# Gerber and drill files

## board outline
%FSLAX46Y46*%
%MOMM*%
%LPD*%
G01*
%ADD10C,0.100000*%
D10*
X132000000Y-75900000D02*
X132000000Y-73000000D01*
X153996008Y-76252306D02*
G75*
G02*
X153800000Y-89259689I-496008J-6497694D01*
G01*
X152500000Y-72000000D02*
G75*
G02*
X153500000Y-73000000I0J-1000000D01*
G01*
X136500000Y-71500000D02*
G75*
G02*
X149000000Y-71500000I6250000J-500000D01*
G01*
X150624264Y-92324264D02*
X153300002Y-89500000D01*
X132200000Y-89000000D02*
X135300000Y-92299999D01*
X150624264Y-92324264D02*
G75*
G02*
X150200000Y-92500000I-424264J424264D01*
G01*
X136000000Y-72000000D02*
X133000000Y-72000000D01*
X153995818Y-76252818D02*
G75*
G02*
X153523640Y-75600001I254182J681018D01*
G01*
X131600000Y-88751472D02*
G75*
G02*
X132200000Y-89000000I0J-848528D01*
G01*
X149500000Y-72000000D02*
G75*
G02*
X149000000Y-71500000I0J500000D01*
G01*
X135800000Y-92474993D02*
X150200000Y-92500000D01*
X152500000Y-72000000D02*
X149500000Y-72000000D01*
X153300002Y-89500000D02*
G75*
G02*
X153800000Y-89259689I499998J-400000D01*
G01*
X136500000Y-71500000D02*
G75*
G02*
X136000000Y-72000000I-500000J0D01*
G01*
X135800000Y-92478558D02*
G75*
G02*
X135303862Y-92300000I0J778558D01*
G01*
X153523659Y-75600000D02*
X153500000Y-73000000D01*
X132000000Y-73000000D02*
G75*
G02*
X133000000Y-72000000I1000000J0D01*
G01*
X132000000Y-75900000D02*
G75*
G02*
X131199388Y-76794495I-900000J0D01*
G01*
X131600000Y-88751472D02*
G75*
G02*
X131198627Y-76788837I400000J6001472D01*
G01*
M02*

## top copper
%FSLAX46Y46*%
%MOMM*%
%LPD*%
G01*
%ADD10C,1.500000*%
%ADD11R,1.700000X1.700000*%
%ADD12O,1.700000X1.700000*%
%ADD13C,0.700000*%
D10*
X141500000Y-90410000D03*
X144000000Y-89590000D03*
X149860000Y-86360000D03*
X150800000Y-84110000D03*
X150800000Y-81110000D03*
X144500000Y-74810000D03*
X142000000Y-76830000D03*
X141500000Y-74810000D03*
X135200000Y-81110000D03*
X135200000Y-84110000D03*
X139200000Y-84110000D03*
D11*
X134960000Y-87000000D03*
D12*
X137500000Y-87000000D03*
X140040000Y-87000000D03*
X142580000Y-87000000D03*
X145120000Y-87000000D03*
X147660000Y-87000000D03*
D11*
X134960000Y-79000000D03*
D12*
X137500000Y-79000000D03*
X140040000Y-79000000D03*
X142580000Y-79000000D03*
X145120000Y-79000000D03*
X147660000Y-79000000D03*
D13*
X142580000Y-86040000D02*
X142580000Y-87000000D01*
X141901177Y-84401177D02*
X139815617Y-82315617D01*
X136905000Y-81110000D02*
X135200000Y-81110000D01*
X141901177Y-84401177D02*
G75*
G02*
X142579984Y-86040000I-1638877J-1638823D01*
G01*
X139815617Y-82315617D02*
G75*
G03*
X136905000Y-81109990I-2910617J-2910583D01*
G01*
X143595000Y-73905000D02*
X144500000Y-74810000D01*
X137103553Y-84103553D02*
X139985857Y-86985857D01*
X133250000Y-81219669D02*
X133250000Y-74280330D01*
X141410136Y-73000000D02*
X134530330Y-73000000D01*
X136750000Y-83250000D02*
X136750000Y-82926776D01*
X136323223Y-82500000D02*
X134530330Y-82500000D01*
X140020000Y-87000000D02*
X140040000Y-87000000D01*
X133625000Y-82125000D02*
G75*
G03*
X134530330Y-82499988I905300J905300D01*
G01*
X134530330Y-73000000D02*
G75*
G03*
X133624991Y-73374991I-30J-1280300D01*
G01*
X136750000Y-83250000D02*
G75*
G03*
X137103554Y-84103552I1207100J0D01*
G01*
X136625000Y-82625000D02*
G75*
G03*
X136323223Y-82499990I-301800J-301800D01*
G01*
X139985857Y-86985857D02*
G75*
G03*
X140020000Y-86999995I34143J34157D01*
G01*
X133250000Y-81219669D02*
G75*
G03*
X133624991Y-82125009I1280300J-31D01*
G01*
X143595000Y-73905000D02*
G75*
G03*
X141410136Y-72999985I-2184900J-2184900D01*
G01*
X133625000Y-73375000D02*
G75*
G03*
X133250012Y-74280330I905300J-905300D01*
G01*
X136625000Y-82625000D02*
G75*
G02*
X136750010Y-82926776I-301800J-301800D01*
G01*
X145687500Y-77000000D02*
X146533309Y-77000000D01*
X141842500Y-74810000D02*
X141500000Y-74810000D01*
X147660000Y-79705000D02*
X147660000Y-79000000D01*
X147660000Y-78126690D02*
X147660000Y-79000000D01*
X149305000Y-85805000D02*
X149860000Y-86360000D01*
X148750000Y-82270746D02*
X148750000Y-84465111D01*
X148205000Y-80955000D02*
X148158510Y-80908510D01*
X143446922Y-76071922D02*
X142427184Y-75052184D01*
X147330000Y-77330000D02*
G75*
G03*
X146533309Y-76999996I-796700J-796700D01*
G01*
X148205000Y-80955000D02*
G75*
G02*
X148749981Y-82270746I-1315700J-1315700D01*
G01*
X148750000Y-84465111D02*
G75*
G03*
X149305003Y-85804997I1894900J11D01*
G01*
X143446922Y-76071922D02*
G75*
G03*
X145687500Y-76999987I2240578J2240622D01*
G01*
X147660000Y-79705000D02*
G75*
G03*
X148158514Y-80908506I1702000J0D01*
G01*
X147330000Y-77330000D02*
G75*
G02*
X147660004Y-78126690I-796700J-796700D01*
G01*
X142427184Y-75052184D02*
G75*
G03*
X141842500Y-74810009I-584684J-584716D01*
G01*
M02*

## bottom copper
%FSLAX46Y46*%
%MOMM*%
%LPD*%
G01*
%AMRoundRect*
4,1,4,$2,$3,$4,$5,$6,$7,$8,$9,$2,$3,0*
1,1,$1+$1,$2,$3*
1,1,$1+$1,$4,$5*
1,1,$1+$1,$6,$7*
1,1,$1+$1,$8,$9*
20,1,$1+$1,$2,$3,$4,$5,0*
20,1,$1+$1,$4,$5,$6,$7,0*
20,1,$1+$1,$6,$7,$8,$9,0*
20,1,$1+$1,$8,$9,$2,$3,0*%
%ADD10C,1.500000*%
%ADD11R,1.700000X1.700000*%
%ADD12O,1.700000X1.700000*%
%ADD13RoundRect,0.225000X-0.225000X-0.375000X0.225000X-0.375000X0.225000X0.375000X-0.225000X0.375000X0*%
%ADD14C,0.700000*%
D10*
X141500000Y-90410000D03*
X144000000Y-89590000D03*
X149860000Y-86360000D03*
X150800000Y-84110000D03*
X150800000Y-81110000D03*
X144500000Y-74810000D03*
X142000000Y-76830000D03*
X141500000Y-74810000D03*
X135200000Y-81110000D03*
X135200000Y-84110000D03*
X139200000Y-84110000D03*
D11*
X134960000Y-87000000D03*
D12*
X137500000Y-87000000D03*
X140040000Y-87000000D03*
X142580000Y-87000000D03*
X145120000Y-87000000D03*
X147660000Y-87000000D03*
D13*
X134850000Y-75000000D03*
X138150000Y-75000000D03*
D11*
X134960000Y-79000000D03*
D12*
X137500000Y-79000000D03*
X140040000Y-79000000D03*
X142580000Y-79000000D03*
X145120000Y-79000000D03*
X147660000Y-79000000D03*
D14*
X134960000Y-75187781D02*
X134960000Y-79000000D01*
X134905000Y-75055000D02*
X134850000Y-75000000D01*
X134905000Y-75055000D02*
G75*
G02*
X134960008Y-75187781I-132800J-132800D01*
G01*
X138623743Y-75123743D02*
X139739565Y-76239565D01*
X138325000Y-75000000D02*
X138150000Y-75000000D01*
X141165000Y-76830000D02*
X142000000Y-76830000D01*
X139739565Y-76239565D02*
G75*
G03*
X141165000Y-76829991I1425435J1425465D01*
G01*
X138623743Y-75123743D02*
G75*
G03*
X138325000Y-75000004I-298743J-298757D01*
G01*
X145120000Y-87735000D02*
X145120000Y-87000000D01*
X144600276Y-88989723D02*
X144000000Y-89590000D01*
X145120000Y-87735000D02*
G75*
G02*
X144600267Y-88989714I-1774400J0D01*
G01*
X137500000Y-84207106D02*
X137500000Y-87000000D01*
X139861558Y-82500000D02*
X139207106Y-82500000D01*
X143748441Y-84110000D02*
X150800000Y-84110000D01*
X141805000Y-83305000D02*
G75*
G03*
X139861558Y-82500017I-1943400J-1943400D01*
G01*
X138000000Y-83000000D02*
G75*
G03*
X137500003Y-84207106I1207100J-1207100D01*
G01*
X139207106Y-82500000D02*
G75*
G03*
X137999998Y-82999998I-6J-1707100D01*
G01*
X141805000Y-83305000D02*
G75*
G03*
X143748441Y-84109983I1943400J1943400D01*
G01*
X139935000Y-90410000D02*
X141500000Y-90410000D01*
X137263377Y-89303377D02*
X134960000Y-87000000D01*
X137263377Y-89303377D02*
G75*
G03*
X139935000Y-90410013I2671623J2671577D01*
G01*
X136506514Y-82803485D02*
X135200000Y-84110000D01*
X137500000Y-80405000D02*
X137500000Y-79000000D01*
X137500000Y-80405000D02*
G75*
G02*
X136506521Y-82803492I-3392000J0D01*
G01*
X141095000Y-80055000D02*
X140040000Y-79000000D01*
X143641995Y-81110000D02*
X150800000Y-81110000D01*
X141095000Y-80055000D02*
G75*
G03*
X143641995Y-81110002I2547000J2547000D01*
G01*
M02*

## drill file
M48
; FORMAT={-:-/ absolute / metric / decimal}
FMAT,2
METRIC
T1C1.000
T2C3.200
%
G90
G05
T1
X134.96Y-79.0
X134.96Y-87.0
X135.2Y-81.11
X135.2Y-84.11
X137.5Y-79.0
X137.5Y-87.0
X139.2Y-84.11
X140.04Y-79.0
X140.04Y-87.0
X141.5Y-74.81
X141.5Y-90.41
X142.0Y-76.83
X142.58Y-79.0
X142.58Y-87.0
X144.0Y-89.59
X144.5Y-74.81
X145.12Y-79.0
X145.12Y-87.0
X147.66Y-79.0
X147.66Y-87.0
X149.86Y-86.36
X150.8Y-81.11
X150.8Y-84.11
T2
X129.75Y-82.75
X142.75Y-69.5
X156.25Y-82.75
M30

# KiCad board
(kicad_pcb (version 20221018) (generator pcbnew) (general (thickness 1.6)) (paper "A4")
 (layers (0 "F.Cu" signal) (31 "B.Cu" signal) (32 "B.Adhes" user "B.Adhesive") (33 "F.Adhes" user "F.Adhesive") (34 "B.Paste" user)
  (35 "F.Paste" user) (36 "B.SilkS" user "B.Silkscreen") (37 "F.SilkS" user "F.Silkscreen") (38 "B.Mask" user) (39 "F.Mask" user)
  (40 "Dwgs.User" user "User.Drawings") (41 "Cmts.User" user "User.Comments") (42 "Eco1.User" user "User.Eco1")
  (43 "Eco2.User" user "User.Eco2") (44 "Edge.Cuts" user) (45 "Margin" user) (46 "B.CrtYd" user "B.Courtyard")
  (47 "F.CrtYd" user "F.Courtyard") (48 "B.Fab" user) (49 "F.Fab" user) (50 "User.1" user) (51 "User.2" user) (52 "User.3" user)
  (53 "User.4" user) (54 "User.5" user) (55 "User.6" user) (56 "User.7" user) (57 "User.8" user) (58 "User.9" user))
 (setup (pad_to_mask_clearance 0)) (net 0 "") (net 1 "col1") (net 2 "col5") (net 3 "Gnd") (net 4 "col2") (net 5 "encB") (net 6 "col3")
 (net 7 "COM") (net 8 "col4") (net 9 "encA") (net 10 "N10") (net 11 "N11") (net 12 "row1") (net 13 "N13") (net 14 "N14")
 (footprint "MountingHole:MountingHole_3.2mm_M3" (layer "F.Cu") (at 129.75 82.75)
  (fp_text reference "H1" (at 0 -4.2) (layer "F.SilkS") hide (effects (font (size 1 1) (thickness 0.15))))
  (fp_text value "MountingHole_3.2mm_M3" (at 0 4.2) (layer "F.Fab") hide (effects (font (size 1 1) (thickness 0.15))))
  (pad "" np_thru_hole circle (at 0 0) (size 3.2 3.2) (drill 3.2) (layers "*.Cu" "*.Mask")))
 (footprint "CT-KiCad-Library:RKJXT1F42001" (layer "F.Cu") (at 143 82.61)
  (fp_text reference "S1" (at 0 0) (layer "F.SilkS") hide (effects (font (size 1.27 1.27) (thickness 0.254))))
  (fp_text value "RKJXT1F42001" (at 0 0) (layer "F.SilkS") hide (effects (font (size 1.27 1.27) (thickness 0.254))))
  (pad "1" thru_hole circle (at -1.5 7.8) (size 1.5 1.5) (drill 1) (layers "*.Cu" "*.Mask") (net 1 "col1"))
  (pad "2" thru_hole circle (at 1 6.98) (size 1.5 1.5) (drill 1) (layers "*.Cu" "*.Mask") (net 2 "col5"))
  (pad "3" thru_hole circle (at 6.86 3.75) (size 1.5 1.5) (drill 1) (layers "*.Cu" "*.Mask") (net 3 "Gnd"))
  (pad "4" thru_hole circle (at 7.8 1.5) (size 1.5 1.5) (drill 1) (layers "*.Cu" "*.Mask") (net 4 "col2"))
  (pad "5" thru_hole circle (at 7.8 -1.5) (size 1.5 1.5) (drill 1) (layers "*.Cu" "*.Mask") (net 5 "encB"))
  (pad "6" thru_hole circle (at 1.5 -7.8) (size 1.5 1.5) (drill 1) (layers "*.Cu" "*.Mask") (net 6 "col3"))
  (pad "7" thru_hole circle (at -1 -5.78) (size 1.5 1.5) (drill 1) (layers "*.Cu" "*.Mask") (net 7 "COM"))
  (pad "8" thru_hole circle (at -1.5 -7.8) (size 1.5 1.5) (drill 1) (layers "*.Cu" "*.Mask") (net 3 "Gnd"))
  (pad "9" thru_hole circle (at -7.8 -1.5) (size 1.5 1.5) (drill 1) (layers "*.Cu" "*.Mask") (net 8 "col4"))
  (pad "10" thru_hole circle (at -7.8 1.5) (size 1.5 1.5) (drill 1) (layers "*.Cu" "*.Mask") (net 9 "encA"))
  (pad "11" thru_hole circle (at -3.8 1.5) (size 1.5 1.5) (drill 1) (layers "*.Cu" "*.Mask") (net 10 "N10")))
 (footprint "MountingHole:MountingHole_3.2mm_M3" (layer "F.Cu") (at 142.75 69.5)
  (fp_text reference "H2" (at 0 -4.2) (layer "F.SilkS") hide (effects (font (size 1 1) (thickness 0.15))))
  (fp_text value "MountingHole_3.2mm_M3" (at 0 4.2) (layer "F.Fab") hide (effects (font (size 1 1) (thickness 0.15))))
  (pad "" np_thru_hole circle (at 0 0) (size 3.2 3.2) (drill 3.2) (layers "*.Cu" "*.Mask")))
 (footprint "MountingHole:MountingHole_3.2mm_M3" (layer "F.Cu") (at 156.25 82.75)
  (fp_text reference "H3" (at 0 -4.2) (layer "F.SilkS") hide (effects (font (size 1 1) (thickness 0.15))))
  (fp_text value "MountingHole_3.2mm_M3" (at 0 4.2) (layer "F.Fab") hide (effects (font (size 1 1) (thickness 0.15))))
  (pad "" np_thru_hole circle (at 0 0) (size 3.2 3.2) (drill 3.2) (layers "*.Cu" "*.Mask")))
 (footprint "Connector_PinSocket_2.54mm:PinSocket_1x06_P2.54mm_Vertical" (layer "B.Cu") (at 134.96 87 -90)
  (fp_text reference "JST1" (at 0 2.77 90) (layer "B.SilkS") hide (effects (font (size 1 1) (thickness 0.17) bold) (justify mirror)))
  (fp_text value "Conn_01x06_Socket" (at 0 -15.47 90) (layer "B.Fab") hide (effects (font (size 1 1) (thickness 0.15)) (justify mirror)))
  (pad "1" thru_hole rect (at 0 0 270) (size 1.7 1.7) (drill 1) (layers "*.Cu" "*.Mask") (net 1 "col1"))
  (pad "2" thru_hole oval (at 0 -2.54 270) (size 1.7 1.7) (drill 1) (layers "*.Cu" "*.Mask") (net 4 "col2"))
  (pad "3" thru_hole oval (at 0 -5.08 270) (size 1.7 1.7) (drill 1) (layers "*.Cu" "*.Mask") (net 6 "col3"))
  (pad "4" thru_hole oval (at 0 -7.62 270) (size 1.7 1.7) (drill 1) (layers "*.Cu" "*.Mask") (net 8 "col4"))
  (pad "5" thru_hole oval (at 0 -10.16 270) (size 1.7 1.7) (drill 1) (layers "*.Cu" "*.Mask") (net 2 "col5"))
  (pad "6" thru_hole oval (at 0 -12.7 270) (size 1.7 1.7) (drill 1) (layers "*.Cu" "*.Mask") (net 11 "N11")))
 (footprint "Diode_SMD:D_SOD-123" (layer "B.Cu") (at 136.5 75)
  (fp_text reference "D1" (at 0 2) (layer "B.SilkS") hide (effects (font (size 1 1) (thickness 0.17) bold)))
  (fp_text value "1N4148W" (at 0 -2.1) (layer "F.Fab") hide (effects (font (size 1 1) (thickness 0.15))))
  (pad "1" smd roundrect (at -1.65 0) (size 0.9 1.2) (layers "B.Cu" "B.Paste" "B.Mask") (roundrect_rratio 0.25) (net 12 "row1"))
  (pad "2" smd roundrect (at 1.65 0) (size 0.9 1.2) (layers "B.Cu" "B.Paste" "B.Mask") (roundrect_rratio 0.25) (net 7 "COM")))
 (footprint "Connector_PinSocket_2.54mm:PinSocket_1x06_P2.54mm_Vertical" (layer "B.Cu") (at 134.96 79 -90)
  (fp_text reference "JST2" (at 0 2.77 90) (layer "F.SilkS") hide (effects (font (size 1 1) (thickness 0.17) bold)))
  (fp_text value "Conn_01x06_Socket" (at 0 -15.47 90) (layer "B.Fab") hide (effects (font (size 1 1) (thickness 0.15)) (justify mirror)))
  (pad "1" thru_hole rect (at 0 0 270) (size 1.7 1.7) (drill 1) (layers "*.Cu" "*.Mask") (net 12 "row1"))
  (pad "2" thru_hole oval (at 0 -2.54 270) (size 1.7 1.7) (drill 1) (layers "*.Cu" "*.Mask") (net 9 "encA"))
  (pad "3" thru_hole oval (at 0 -5.08 270) (size 1.7 1.7) (drill 1) (layers "*.Cu" "*.Mask") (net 5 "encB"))
  (pad "4" thru_hole oval (at 0 -7.62 270) (size 1.7 1.7) (drill 1) (layers "*.Cu" "*.Mask") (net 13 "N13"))
  (pad "5" thru_hole oval (at 0 -10.16 270) (size 1.7 1.7) (drill 1) (layers "*.Cu" "*.Mask") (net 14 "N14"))
  (pad "6" thru_hole oval (at 0 -12.7 270) (size 1.7 1.7) (drill 1) (layers "*.Cu" "*.Mask") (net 3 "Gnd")))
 (gr_line (start 132 75.9) (end 132 73) (stroke (width 0.1) (type default)) (layer "Edge.Cuts"))
 (gr_arc (start 153.996008 76.252306) (mid 160.015858 82.848187) (end 153.8 89.259689) (stroke (width 0.1) (type default))
  (layer "Edge.Cuts"))
 (gr_arc (start 152.5 72) (mid 153.207107 72.292893) (end 153.5 73) (stroke (width 0.1) (type default)) (layer "Edge.Cuts"))
 (gr_arc (start 136.5 71.5) (mid 142.75 65.730032) (end 149 71.5) (stroke (width 0.1) (type default)) (layer "Edge.Cuts"))
 (gr_line (start 150.624264 92.324264) (end 153.300002 89.5) (stroke (width 0.1) (type default)) (layer "Edge.Cuts"))
 (gr_line (start 132.2 89) (end 135.3 92.299999) (stroke (width 0.1) (type default)) (layer "Edge.Cuts"))
 (gr_arc (start 150.624264 92.324264) (mid 150.42961 92.454328) (end 150.2 92.5) (stroke (width 0.1) (type default)) (layer "Edge.Cuts"))
 (gr_line (start 136 72) (end 133 72) (stroke (width 0.1) (type default)) (layer "Edge.Cuts"))
 (gr_arc (start 153.995818 76.252818) (mid 153.661019 75.997809) (end 153.523659 75.6) (stroke (width 0.1) (type default))
  (layer "Edge.Cuts"))
 (gr_arc (start 131.6 88.751472) (mid 131.924718 88.816062) (end 132.2 89) (stroke (width 0.1) (type default)) (layer "Edge.Cuts"))
 (gr_arc (start 149.5 72) (mid 149.146447 71.853553) (end 149 71.5) (stroke (width 0.1) (type default)) (layer "Edge.Cuts"))
 (gr_line (start 135.8 92.474993) (end 150.2 92.5) (stroke (width 0.1) (type default)) (layer "Edge.Cuts"))
 (gr_line (start 152.5 72) (end 149.5 72) (stroke (width 0.1) (type default)) (layer "Edge.Cuts"))
 (gr_arc (start 153.300002 89.5) (mid 153.522625 89.322885) (end 153.8 89.259689) (stroke (width 0.1) (type default)) (layer "Edge.Cuts"))
 (gr_arc (start 136.5 71.5) (mid 136.353553 71.853553) (end 136 72) (stroke (width 0.1) (type default)) (layer "Edge.Cuts"))
 (gr_arc (start 135.8 92.478558) (mid 135.536355 92.43256) (end 135.303862 92.3) (stroke (width 0.1) (type default)) (layer "Edge.Cuts"))
 (gr_line (start 153.523659 75.6) (end 153.5 73) (stroke (width 0.1) (type default)) (layer "Edge.Cuts"))
 (gr_arc (start 132 73) (mid 132.292893 72.292893) (end 133 72) (stroke (width 0.1) (type default)) (layer "Edge.Cuts"))
 (gr_arc (start 132 75.9) (mid 131.770615 76.500229) (end 131.199388 76.794495) (stroke (width 0.1) (type default)) (layer "Edge.Cuts"))
 (gr_arc (start 131.6 88.751472) (mid 125.988595 82.951696) (end 131.198627 76.788837) (stroke (width 0.1) (type default))
  (layer "Edge.Cuts"))
 (segment (start 134.96 75.187781) (end 134.96 79) (width 0.7) (layer "B.Cu") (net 12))
 (segment (start 134.905 75.055) (end 134.85 75) (width 0.7) (layer "B.Cu") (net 12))
 (arc (start 134.905 75.055) (mid 134.945705 75.11592) (end 134.96 75.187781) (width 0.7) (layer "B.Cu") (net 12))
 (segment (start 138.623743 75.123743) (end 139.739565 76.239565) (width 0.7) (layer "B.Cu") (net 7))
 (segment (start 138.325 75) (end 138.15 75) (width 0.7) (layer "B.Cu") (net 7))
 (segment (start 141.165 76.83) (end 142 76.83) (width 0.7) (layer "B.Cu") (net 7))
 (arc (start 139.739565 76.239565) (mid 140.39356 76.67655) (end 141.165 76.83) (width 0.7) (layer "B.Cu") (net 7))
 (arc (start 138.623743 75.123743) (mid 138.486678 75.032159) (end 138.325 75) (width 0.7) (layer "B.Cu") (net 7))
 (segment (start 145.12 87.735) (end 145.12 87) (width 0.7) (layer "B.Cu") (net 2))
 (segment (start 144.600276 88.989723) (end 144 89.59) (width 0.7) (layer "B.Cu") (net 2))
 (arc (start 145.12 87.735) (mid 144.984928 88.414051) (end 144.600276 88.989723) (width 0.7) (layer "B.Cu") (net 2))
 (segment (start 142.58 86.04) (end 142.58 87) (width 0.7) (layer "F.Cu") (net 8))
 (segment (start 141.901177 84.401177) (end 139.815617 82.315617) (width 0.7) (layer "F.Cu") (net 8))
 (segment (start 136.905 81.11) (end 135.2 81.11) (width 0.7) (layer "F.Cu") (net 8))
 (arc (start 141.901177 84.401177) (mid 142.403579 85.153075) (end 142.58 86.04) (width 0.7) (layer "F.Cu") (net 8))
 (arc (start 139.815617 82.315617) (mid 138.480214 81.423329) (end 136.905 81.11) (width 0.7) (layer "F.Cu") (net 8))
 (segment (start 143.595 73.905) (end 144.5 74.81) (width 0.7) (layer "F.Cu") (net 6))
 (segment (start 137.103553 84.103553) (end 139.985857 86.985857) (width 0.7) (layer "F.Cu") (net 6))
 (segment (start 133.25 81.219669) (end 133.25 74.28033) (width 0.7) (layer "F.Cu") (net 6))
 (segment (start 141.410136 73) (end 134.53033 73) (width 0.7) (layer "F.Cu") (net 6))
 (segment (start 136.75 83.25) (end 136.75 82.926776) (width 0.7) (layer "F.Cu") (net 6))
 (segment (start 136.323223 82.5) (end 134.53033 82.5) (width 0.7) (layer "F.Cu") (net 6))
 (segment (start 140.02 87) (end 140.04 87) (width 0.7) (layer "F.Cu") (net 6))
 (arc (start 133.625 82.125) (mid 134.040368 82.40254) (end 134.53033 82.5) (width 0.7) (layer "F.Cu") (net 6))
 (arc (start 134.53033 73) (mid 134.040368 73.097459) (end 133.625 73.375) (width 0.7) (layer "F.Cu") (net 6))
 (arc (start 136.75 83.25) (mid 136.841885 83.711939) (end 137.103553 84.103553) (width 0.7) (layer "F.Cu") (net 6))
 (arc (start 136.625 82.625) (mid 136.486543 82.532486) (end 136.323223 82.5) (width 0.7) (layer "F.Cu") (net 6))
 (arc (start 139.985857 86.985857) (mid 140.001522 86.996324) (end 140.02 87) (width 0.7) (layer "F.Cu") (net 6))
 (arc (start 133.25 81.219669) (mid 133.347459 81.70963) (end 133.625 82.125) (width 0.7) (layer "F.Cu") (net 6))
 (arc (start 143.595 73.905) (mid 142.592576 73.235201) (end 141.410136 73) (width 0.7) (layer "F.Cu") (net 6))
 (arc (start 133.625 73.375) (mid 133.347459 73.790368) (end 133.25 74.28033) (width 0.7) (layer "F.Cu") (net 6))
 (arc (start 136.625 82.625) (mid 136.717513 82.763456) (end 136.75 82.926776) (width 0.7) (layer "F.Cu") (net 6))
 (segment (start 137.5 84.207106) (end 137.5 87) (width 0.7) (layer "B.Cu") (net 4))
 (segment (start 139.861558 82.5) (end 139.207106 82.5) (width 0.7) (layer "B.Cu") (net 4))
 (segment (start 143.748441 84.11) (end 150.8 84.11) (width 0.7) (layer "B.Cu") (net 4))
 (arc (start 141.805 83.305) (mid 140.913341 82.709212) (end 139.861558 82.5) (width 0.7) (layer "B.Cu") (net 4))
 (arc (start 138 83) (mid 137.629945 83.553825) (end 137.5 84.207106) (width 0.7) (layer "B.Cu") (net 4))
 (arc (start 139.207106 82.5) (mid 138.553825 82.629945) (end 138 83) (width 0.7) (layer "B.Cu") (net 4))
 (arc (start 141.805 83.305) (mid 142.696658 83.900787) (end 143.748441 84.11) (width 0.7) (layer "B.Cu") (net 4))
 (segment (start 139.935 90.41) (end 141.5 90.41) (width 0.7) (layer "B.Cu") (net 1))
 (segment (start 137.263377 89.303377) (end 134.96 87) (width 0.7) (layer "B.Cu") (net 1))
 (arc (start 137.263377 89.303377) (mid 138.489128 90.122398) (end 139.935 90.41) (width 0.7) (layer "B.Cu") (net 1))
 (segment (start 136.506514 82.803485) (end 135.2 84.11) (width 0.7) (layer "B.Cu") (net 9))
 (segment (start 137.5 80.405) (end 137.5 79) (width 0.7) (layer "B.Cu") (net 9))
 (arc (start 137.5 80.405) (mid 137.241801 81.70305) (end 136.506514 82.803485) (width 0.7) (layer "B.Cu") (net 9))
 (segment (start 141.095 80.055) (end 140.04 79) (width 0.7) (layer "B.Cu") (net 5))
 (segment (start 143.641995 81.11) (end 150.8 81.11) (width 0.7) (layer "B.Cu") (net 5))
 (arc (start 141.095 80.055) (mid 142.263571 80.835814) (end 143.641995 81.11) (width 0.7) (layer "B.Cu") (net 5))
 (segment (start 145.6875 77) (end 146.533309 77) (width 0.7) (layer "F.Cu") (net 3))
 (segment (start 141.8425 74.81) (end 141.5 74.81) (width 0.7) (layer "F.Cu") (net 3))
 (segment (start 147.66 79.705) (end 147.66 79) (width 0.7) (layer "F.Cu") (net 3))
 (segment (start 147.66 78.12669) (end 147.66 79) (width 0.7) (layer "F.Cu") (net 3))
 (segment (start 149.305 85.805) (end 149.86 86.36) (width 0.7) (layer "F.Cu") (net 3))
 (segment (start 148.75 82.270746) (end 148.75 84.465111) (width 0.7) (layer "F.Cu") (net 3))
 (segment (start 148.205 80.955) (end 148.15851 80.90851) (width 0.7) (layer "F.Cu") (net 3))
 (segment (start 143.446922 76.071922) (end 142.427184 75.052184) (width 0.7) (layer "F.Cu") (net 3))
 (arc (start 147.33 77.33) (mid 146.964475 77.085764) (end 146.533309 77) (width 0.7) (layer "F.Cu") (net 3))
 (arc (start 148.205 80.955) (mid 148.608359 81.558669) (end 148.75 82.270746) (width 0.7) (layer "F.Cu") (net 3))
 (arc (start 148.75 84.465111) (mid 148.894239 85.190253) (end 149.305 85.805) (width 0.7) (layer "F.Cu") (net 3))
 (arc (start 143.446922 76.071922) (mid 144.474908 76.7588) (end 145.6875 77) (width 0.7) (layer "F.Cu") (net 3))
 (arc (start 147.66 79.705) (mid 147.789558 80.356334) (end 148.15851 80.90851) (width 0.7) (layer "F.Cu") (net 3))
 (arc (start 147.33 77.33) (mid 147.574235 77.695524) (end 147.66 78.12669) (width 0.7) (layer "F.Cu") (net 3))
 (arc (start 142.427184 75.052184) (mid 142.158928 74.872941) (end 141.8425 74.81) (width 0.7) (layer "F.Cu") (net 3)))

